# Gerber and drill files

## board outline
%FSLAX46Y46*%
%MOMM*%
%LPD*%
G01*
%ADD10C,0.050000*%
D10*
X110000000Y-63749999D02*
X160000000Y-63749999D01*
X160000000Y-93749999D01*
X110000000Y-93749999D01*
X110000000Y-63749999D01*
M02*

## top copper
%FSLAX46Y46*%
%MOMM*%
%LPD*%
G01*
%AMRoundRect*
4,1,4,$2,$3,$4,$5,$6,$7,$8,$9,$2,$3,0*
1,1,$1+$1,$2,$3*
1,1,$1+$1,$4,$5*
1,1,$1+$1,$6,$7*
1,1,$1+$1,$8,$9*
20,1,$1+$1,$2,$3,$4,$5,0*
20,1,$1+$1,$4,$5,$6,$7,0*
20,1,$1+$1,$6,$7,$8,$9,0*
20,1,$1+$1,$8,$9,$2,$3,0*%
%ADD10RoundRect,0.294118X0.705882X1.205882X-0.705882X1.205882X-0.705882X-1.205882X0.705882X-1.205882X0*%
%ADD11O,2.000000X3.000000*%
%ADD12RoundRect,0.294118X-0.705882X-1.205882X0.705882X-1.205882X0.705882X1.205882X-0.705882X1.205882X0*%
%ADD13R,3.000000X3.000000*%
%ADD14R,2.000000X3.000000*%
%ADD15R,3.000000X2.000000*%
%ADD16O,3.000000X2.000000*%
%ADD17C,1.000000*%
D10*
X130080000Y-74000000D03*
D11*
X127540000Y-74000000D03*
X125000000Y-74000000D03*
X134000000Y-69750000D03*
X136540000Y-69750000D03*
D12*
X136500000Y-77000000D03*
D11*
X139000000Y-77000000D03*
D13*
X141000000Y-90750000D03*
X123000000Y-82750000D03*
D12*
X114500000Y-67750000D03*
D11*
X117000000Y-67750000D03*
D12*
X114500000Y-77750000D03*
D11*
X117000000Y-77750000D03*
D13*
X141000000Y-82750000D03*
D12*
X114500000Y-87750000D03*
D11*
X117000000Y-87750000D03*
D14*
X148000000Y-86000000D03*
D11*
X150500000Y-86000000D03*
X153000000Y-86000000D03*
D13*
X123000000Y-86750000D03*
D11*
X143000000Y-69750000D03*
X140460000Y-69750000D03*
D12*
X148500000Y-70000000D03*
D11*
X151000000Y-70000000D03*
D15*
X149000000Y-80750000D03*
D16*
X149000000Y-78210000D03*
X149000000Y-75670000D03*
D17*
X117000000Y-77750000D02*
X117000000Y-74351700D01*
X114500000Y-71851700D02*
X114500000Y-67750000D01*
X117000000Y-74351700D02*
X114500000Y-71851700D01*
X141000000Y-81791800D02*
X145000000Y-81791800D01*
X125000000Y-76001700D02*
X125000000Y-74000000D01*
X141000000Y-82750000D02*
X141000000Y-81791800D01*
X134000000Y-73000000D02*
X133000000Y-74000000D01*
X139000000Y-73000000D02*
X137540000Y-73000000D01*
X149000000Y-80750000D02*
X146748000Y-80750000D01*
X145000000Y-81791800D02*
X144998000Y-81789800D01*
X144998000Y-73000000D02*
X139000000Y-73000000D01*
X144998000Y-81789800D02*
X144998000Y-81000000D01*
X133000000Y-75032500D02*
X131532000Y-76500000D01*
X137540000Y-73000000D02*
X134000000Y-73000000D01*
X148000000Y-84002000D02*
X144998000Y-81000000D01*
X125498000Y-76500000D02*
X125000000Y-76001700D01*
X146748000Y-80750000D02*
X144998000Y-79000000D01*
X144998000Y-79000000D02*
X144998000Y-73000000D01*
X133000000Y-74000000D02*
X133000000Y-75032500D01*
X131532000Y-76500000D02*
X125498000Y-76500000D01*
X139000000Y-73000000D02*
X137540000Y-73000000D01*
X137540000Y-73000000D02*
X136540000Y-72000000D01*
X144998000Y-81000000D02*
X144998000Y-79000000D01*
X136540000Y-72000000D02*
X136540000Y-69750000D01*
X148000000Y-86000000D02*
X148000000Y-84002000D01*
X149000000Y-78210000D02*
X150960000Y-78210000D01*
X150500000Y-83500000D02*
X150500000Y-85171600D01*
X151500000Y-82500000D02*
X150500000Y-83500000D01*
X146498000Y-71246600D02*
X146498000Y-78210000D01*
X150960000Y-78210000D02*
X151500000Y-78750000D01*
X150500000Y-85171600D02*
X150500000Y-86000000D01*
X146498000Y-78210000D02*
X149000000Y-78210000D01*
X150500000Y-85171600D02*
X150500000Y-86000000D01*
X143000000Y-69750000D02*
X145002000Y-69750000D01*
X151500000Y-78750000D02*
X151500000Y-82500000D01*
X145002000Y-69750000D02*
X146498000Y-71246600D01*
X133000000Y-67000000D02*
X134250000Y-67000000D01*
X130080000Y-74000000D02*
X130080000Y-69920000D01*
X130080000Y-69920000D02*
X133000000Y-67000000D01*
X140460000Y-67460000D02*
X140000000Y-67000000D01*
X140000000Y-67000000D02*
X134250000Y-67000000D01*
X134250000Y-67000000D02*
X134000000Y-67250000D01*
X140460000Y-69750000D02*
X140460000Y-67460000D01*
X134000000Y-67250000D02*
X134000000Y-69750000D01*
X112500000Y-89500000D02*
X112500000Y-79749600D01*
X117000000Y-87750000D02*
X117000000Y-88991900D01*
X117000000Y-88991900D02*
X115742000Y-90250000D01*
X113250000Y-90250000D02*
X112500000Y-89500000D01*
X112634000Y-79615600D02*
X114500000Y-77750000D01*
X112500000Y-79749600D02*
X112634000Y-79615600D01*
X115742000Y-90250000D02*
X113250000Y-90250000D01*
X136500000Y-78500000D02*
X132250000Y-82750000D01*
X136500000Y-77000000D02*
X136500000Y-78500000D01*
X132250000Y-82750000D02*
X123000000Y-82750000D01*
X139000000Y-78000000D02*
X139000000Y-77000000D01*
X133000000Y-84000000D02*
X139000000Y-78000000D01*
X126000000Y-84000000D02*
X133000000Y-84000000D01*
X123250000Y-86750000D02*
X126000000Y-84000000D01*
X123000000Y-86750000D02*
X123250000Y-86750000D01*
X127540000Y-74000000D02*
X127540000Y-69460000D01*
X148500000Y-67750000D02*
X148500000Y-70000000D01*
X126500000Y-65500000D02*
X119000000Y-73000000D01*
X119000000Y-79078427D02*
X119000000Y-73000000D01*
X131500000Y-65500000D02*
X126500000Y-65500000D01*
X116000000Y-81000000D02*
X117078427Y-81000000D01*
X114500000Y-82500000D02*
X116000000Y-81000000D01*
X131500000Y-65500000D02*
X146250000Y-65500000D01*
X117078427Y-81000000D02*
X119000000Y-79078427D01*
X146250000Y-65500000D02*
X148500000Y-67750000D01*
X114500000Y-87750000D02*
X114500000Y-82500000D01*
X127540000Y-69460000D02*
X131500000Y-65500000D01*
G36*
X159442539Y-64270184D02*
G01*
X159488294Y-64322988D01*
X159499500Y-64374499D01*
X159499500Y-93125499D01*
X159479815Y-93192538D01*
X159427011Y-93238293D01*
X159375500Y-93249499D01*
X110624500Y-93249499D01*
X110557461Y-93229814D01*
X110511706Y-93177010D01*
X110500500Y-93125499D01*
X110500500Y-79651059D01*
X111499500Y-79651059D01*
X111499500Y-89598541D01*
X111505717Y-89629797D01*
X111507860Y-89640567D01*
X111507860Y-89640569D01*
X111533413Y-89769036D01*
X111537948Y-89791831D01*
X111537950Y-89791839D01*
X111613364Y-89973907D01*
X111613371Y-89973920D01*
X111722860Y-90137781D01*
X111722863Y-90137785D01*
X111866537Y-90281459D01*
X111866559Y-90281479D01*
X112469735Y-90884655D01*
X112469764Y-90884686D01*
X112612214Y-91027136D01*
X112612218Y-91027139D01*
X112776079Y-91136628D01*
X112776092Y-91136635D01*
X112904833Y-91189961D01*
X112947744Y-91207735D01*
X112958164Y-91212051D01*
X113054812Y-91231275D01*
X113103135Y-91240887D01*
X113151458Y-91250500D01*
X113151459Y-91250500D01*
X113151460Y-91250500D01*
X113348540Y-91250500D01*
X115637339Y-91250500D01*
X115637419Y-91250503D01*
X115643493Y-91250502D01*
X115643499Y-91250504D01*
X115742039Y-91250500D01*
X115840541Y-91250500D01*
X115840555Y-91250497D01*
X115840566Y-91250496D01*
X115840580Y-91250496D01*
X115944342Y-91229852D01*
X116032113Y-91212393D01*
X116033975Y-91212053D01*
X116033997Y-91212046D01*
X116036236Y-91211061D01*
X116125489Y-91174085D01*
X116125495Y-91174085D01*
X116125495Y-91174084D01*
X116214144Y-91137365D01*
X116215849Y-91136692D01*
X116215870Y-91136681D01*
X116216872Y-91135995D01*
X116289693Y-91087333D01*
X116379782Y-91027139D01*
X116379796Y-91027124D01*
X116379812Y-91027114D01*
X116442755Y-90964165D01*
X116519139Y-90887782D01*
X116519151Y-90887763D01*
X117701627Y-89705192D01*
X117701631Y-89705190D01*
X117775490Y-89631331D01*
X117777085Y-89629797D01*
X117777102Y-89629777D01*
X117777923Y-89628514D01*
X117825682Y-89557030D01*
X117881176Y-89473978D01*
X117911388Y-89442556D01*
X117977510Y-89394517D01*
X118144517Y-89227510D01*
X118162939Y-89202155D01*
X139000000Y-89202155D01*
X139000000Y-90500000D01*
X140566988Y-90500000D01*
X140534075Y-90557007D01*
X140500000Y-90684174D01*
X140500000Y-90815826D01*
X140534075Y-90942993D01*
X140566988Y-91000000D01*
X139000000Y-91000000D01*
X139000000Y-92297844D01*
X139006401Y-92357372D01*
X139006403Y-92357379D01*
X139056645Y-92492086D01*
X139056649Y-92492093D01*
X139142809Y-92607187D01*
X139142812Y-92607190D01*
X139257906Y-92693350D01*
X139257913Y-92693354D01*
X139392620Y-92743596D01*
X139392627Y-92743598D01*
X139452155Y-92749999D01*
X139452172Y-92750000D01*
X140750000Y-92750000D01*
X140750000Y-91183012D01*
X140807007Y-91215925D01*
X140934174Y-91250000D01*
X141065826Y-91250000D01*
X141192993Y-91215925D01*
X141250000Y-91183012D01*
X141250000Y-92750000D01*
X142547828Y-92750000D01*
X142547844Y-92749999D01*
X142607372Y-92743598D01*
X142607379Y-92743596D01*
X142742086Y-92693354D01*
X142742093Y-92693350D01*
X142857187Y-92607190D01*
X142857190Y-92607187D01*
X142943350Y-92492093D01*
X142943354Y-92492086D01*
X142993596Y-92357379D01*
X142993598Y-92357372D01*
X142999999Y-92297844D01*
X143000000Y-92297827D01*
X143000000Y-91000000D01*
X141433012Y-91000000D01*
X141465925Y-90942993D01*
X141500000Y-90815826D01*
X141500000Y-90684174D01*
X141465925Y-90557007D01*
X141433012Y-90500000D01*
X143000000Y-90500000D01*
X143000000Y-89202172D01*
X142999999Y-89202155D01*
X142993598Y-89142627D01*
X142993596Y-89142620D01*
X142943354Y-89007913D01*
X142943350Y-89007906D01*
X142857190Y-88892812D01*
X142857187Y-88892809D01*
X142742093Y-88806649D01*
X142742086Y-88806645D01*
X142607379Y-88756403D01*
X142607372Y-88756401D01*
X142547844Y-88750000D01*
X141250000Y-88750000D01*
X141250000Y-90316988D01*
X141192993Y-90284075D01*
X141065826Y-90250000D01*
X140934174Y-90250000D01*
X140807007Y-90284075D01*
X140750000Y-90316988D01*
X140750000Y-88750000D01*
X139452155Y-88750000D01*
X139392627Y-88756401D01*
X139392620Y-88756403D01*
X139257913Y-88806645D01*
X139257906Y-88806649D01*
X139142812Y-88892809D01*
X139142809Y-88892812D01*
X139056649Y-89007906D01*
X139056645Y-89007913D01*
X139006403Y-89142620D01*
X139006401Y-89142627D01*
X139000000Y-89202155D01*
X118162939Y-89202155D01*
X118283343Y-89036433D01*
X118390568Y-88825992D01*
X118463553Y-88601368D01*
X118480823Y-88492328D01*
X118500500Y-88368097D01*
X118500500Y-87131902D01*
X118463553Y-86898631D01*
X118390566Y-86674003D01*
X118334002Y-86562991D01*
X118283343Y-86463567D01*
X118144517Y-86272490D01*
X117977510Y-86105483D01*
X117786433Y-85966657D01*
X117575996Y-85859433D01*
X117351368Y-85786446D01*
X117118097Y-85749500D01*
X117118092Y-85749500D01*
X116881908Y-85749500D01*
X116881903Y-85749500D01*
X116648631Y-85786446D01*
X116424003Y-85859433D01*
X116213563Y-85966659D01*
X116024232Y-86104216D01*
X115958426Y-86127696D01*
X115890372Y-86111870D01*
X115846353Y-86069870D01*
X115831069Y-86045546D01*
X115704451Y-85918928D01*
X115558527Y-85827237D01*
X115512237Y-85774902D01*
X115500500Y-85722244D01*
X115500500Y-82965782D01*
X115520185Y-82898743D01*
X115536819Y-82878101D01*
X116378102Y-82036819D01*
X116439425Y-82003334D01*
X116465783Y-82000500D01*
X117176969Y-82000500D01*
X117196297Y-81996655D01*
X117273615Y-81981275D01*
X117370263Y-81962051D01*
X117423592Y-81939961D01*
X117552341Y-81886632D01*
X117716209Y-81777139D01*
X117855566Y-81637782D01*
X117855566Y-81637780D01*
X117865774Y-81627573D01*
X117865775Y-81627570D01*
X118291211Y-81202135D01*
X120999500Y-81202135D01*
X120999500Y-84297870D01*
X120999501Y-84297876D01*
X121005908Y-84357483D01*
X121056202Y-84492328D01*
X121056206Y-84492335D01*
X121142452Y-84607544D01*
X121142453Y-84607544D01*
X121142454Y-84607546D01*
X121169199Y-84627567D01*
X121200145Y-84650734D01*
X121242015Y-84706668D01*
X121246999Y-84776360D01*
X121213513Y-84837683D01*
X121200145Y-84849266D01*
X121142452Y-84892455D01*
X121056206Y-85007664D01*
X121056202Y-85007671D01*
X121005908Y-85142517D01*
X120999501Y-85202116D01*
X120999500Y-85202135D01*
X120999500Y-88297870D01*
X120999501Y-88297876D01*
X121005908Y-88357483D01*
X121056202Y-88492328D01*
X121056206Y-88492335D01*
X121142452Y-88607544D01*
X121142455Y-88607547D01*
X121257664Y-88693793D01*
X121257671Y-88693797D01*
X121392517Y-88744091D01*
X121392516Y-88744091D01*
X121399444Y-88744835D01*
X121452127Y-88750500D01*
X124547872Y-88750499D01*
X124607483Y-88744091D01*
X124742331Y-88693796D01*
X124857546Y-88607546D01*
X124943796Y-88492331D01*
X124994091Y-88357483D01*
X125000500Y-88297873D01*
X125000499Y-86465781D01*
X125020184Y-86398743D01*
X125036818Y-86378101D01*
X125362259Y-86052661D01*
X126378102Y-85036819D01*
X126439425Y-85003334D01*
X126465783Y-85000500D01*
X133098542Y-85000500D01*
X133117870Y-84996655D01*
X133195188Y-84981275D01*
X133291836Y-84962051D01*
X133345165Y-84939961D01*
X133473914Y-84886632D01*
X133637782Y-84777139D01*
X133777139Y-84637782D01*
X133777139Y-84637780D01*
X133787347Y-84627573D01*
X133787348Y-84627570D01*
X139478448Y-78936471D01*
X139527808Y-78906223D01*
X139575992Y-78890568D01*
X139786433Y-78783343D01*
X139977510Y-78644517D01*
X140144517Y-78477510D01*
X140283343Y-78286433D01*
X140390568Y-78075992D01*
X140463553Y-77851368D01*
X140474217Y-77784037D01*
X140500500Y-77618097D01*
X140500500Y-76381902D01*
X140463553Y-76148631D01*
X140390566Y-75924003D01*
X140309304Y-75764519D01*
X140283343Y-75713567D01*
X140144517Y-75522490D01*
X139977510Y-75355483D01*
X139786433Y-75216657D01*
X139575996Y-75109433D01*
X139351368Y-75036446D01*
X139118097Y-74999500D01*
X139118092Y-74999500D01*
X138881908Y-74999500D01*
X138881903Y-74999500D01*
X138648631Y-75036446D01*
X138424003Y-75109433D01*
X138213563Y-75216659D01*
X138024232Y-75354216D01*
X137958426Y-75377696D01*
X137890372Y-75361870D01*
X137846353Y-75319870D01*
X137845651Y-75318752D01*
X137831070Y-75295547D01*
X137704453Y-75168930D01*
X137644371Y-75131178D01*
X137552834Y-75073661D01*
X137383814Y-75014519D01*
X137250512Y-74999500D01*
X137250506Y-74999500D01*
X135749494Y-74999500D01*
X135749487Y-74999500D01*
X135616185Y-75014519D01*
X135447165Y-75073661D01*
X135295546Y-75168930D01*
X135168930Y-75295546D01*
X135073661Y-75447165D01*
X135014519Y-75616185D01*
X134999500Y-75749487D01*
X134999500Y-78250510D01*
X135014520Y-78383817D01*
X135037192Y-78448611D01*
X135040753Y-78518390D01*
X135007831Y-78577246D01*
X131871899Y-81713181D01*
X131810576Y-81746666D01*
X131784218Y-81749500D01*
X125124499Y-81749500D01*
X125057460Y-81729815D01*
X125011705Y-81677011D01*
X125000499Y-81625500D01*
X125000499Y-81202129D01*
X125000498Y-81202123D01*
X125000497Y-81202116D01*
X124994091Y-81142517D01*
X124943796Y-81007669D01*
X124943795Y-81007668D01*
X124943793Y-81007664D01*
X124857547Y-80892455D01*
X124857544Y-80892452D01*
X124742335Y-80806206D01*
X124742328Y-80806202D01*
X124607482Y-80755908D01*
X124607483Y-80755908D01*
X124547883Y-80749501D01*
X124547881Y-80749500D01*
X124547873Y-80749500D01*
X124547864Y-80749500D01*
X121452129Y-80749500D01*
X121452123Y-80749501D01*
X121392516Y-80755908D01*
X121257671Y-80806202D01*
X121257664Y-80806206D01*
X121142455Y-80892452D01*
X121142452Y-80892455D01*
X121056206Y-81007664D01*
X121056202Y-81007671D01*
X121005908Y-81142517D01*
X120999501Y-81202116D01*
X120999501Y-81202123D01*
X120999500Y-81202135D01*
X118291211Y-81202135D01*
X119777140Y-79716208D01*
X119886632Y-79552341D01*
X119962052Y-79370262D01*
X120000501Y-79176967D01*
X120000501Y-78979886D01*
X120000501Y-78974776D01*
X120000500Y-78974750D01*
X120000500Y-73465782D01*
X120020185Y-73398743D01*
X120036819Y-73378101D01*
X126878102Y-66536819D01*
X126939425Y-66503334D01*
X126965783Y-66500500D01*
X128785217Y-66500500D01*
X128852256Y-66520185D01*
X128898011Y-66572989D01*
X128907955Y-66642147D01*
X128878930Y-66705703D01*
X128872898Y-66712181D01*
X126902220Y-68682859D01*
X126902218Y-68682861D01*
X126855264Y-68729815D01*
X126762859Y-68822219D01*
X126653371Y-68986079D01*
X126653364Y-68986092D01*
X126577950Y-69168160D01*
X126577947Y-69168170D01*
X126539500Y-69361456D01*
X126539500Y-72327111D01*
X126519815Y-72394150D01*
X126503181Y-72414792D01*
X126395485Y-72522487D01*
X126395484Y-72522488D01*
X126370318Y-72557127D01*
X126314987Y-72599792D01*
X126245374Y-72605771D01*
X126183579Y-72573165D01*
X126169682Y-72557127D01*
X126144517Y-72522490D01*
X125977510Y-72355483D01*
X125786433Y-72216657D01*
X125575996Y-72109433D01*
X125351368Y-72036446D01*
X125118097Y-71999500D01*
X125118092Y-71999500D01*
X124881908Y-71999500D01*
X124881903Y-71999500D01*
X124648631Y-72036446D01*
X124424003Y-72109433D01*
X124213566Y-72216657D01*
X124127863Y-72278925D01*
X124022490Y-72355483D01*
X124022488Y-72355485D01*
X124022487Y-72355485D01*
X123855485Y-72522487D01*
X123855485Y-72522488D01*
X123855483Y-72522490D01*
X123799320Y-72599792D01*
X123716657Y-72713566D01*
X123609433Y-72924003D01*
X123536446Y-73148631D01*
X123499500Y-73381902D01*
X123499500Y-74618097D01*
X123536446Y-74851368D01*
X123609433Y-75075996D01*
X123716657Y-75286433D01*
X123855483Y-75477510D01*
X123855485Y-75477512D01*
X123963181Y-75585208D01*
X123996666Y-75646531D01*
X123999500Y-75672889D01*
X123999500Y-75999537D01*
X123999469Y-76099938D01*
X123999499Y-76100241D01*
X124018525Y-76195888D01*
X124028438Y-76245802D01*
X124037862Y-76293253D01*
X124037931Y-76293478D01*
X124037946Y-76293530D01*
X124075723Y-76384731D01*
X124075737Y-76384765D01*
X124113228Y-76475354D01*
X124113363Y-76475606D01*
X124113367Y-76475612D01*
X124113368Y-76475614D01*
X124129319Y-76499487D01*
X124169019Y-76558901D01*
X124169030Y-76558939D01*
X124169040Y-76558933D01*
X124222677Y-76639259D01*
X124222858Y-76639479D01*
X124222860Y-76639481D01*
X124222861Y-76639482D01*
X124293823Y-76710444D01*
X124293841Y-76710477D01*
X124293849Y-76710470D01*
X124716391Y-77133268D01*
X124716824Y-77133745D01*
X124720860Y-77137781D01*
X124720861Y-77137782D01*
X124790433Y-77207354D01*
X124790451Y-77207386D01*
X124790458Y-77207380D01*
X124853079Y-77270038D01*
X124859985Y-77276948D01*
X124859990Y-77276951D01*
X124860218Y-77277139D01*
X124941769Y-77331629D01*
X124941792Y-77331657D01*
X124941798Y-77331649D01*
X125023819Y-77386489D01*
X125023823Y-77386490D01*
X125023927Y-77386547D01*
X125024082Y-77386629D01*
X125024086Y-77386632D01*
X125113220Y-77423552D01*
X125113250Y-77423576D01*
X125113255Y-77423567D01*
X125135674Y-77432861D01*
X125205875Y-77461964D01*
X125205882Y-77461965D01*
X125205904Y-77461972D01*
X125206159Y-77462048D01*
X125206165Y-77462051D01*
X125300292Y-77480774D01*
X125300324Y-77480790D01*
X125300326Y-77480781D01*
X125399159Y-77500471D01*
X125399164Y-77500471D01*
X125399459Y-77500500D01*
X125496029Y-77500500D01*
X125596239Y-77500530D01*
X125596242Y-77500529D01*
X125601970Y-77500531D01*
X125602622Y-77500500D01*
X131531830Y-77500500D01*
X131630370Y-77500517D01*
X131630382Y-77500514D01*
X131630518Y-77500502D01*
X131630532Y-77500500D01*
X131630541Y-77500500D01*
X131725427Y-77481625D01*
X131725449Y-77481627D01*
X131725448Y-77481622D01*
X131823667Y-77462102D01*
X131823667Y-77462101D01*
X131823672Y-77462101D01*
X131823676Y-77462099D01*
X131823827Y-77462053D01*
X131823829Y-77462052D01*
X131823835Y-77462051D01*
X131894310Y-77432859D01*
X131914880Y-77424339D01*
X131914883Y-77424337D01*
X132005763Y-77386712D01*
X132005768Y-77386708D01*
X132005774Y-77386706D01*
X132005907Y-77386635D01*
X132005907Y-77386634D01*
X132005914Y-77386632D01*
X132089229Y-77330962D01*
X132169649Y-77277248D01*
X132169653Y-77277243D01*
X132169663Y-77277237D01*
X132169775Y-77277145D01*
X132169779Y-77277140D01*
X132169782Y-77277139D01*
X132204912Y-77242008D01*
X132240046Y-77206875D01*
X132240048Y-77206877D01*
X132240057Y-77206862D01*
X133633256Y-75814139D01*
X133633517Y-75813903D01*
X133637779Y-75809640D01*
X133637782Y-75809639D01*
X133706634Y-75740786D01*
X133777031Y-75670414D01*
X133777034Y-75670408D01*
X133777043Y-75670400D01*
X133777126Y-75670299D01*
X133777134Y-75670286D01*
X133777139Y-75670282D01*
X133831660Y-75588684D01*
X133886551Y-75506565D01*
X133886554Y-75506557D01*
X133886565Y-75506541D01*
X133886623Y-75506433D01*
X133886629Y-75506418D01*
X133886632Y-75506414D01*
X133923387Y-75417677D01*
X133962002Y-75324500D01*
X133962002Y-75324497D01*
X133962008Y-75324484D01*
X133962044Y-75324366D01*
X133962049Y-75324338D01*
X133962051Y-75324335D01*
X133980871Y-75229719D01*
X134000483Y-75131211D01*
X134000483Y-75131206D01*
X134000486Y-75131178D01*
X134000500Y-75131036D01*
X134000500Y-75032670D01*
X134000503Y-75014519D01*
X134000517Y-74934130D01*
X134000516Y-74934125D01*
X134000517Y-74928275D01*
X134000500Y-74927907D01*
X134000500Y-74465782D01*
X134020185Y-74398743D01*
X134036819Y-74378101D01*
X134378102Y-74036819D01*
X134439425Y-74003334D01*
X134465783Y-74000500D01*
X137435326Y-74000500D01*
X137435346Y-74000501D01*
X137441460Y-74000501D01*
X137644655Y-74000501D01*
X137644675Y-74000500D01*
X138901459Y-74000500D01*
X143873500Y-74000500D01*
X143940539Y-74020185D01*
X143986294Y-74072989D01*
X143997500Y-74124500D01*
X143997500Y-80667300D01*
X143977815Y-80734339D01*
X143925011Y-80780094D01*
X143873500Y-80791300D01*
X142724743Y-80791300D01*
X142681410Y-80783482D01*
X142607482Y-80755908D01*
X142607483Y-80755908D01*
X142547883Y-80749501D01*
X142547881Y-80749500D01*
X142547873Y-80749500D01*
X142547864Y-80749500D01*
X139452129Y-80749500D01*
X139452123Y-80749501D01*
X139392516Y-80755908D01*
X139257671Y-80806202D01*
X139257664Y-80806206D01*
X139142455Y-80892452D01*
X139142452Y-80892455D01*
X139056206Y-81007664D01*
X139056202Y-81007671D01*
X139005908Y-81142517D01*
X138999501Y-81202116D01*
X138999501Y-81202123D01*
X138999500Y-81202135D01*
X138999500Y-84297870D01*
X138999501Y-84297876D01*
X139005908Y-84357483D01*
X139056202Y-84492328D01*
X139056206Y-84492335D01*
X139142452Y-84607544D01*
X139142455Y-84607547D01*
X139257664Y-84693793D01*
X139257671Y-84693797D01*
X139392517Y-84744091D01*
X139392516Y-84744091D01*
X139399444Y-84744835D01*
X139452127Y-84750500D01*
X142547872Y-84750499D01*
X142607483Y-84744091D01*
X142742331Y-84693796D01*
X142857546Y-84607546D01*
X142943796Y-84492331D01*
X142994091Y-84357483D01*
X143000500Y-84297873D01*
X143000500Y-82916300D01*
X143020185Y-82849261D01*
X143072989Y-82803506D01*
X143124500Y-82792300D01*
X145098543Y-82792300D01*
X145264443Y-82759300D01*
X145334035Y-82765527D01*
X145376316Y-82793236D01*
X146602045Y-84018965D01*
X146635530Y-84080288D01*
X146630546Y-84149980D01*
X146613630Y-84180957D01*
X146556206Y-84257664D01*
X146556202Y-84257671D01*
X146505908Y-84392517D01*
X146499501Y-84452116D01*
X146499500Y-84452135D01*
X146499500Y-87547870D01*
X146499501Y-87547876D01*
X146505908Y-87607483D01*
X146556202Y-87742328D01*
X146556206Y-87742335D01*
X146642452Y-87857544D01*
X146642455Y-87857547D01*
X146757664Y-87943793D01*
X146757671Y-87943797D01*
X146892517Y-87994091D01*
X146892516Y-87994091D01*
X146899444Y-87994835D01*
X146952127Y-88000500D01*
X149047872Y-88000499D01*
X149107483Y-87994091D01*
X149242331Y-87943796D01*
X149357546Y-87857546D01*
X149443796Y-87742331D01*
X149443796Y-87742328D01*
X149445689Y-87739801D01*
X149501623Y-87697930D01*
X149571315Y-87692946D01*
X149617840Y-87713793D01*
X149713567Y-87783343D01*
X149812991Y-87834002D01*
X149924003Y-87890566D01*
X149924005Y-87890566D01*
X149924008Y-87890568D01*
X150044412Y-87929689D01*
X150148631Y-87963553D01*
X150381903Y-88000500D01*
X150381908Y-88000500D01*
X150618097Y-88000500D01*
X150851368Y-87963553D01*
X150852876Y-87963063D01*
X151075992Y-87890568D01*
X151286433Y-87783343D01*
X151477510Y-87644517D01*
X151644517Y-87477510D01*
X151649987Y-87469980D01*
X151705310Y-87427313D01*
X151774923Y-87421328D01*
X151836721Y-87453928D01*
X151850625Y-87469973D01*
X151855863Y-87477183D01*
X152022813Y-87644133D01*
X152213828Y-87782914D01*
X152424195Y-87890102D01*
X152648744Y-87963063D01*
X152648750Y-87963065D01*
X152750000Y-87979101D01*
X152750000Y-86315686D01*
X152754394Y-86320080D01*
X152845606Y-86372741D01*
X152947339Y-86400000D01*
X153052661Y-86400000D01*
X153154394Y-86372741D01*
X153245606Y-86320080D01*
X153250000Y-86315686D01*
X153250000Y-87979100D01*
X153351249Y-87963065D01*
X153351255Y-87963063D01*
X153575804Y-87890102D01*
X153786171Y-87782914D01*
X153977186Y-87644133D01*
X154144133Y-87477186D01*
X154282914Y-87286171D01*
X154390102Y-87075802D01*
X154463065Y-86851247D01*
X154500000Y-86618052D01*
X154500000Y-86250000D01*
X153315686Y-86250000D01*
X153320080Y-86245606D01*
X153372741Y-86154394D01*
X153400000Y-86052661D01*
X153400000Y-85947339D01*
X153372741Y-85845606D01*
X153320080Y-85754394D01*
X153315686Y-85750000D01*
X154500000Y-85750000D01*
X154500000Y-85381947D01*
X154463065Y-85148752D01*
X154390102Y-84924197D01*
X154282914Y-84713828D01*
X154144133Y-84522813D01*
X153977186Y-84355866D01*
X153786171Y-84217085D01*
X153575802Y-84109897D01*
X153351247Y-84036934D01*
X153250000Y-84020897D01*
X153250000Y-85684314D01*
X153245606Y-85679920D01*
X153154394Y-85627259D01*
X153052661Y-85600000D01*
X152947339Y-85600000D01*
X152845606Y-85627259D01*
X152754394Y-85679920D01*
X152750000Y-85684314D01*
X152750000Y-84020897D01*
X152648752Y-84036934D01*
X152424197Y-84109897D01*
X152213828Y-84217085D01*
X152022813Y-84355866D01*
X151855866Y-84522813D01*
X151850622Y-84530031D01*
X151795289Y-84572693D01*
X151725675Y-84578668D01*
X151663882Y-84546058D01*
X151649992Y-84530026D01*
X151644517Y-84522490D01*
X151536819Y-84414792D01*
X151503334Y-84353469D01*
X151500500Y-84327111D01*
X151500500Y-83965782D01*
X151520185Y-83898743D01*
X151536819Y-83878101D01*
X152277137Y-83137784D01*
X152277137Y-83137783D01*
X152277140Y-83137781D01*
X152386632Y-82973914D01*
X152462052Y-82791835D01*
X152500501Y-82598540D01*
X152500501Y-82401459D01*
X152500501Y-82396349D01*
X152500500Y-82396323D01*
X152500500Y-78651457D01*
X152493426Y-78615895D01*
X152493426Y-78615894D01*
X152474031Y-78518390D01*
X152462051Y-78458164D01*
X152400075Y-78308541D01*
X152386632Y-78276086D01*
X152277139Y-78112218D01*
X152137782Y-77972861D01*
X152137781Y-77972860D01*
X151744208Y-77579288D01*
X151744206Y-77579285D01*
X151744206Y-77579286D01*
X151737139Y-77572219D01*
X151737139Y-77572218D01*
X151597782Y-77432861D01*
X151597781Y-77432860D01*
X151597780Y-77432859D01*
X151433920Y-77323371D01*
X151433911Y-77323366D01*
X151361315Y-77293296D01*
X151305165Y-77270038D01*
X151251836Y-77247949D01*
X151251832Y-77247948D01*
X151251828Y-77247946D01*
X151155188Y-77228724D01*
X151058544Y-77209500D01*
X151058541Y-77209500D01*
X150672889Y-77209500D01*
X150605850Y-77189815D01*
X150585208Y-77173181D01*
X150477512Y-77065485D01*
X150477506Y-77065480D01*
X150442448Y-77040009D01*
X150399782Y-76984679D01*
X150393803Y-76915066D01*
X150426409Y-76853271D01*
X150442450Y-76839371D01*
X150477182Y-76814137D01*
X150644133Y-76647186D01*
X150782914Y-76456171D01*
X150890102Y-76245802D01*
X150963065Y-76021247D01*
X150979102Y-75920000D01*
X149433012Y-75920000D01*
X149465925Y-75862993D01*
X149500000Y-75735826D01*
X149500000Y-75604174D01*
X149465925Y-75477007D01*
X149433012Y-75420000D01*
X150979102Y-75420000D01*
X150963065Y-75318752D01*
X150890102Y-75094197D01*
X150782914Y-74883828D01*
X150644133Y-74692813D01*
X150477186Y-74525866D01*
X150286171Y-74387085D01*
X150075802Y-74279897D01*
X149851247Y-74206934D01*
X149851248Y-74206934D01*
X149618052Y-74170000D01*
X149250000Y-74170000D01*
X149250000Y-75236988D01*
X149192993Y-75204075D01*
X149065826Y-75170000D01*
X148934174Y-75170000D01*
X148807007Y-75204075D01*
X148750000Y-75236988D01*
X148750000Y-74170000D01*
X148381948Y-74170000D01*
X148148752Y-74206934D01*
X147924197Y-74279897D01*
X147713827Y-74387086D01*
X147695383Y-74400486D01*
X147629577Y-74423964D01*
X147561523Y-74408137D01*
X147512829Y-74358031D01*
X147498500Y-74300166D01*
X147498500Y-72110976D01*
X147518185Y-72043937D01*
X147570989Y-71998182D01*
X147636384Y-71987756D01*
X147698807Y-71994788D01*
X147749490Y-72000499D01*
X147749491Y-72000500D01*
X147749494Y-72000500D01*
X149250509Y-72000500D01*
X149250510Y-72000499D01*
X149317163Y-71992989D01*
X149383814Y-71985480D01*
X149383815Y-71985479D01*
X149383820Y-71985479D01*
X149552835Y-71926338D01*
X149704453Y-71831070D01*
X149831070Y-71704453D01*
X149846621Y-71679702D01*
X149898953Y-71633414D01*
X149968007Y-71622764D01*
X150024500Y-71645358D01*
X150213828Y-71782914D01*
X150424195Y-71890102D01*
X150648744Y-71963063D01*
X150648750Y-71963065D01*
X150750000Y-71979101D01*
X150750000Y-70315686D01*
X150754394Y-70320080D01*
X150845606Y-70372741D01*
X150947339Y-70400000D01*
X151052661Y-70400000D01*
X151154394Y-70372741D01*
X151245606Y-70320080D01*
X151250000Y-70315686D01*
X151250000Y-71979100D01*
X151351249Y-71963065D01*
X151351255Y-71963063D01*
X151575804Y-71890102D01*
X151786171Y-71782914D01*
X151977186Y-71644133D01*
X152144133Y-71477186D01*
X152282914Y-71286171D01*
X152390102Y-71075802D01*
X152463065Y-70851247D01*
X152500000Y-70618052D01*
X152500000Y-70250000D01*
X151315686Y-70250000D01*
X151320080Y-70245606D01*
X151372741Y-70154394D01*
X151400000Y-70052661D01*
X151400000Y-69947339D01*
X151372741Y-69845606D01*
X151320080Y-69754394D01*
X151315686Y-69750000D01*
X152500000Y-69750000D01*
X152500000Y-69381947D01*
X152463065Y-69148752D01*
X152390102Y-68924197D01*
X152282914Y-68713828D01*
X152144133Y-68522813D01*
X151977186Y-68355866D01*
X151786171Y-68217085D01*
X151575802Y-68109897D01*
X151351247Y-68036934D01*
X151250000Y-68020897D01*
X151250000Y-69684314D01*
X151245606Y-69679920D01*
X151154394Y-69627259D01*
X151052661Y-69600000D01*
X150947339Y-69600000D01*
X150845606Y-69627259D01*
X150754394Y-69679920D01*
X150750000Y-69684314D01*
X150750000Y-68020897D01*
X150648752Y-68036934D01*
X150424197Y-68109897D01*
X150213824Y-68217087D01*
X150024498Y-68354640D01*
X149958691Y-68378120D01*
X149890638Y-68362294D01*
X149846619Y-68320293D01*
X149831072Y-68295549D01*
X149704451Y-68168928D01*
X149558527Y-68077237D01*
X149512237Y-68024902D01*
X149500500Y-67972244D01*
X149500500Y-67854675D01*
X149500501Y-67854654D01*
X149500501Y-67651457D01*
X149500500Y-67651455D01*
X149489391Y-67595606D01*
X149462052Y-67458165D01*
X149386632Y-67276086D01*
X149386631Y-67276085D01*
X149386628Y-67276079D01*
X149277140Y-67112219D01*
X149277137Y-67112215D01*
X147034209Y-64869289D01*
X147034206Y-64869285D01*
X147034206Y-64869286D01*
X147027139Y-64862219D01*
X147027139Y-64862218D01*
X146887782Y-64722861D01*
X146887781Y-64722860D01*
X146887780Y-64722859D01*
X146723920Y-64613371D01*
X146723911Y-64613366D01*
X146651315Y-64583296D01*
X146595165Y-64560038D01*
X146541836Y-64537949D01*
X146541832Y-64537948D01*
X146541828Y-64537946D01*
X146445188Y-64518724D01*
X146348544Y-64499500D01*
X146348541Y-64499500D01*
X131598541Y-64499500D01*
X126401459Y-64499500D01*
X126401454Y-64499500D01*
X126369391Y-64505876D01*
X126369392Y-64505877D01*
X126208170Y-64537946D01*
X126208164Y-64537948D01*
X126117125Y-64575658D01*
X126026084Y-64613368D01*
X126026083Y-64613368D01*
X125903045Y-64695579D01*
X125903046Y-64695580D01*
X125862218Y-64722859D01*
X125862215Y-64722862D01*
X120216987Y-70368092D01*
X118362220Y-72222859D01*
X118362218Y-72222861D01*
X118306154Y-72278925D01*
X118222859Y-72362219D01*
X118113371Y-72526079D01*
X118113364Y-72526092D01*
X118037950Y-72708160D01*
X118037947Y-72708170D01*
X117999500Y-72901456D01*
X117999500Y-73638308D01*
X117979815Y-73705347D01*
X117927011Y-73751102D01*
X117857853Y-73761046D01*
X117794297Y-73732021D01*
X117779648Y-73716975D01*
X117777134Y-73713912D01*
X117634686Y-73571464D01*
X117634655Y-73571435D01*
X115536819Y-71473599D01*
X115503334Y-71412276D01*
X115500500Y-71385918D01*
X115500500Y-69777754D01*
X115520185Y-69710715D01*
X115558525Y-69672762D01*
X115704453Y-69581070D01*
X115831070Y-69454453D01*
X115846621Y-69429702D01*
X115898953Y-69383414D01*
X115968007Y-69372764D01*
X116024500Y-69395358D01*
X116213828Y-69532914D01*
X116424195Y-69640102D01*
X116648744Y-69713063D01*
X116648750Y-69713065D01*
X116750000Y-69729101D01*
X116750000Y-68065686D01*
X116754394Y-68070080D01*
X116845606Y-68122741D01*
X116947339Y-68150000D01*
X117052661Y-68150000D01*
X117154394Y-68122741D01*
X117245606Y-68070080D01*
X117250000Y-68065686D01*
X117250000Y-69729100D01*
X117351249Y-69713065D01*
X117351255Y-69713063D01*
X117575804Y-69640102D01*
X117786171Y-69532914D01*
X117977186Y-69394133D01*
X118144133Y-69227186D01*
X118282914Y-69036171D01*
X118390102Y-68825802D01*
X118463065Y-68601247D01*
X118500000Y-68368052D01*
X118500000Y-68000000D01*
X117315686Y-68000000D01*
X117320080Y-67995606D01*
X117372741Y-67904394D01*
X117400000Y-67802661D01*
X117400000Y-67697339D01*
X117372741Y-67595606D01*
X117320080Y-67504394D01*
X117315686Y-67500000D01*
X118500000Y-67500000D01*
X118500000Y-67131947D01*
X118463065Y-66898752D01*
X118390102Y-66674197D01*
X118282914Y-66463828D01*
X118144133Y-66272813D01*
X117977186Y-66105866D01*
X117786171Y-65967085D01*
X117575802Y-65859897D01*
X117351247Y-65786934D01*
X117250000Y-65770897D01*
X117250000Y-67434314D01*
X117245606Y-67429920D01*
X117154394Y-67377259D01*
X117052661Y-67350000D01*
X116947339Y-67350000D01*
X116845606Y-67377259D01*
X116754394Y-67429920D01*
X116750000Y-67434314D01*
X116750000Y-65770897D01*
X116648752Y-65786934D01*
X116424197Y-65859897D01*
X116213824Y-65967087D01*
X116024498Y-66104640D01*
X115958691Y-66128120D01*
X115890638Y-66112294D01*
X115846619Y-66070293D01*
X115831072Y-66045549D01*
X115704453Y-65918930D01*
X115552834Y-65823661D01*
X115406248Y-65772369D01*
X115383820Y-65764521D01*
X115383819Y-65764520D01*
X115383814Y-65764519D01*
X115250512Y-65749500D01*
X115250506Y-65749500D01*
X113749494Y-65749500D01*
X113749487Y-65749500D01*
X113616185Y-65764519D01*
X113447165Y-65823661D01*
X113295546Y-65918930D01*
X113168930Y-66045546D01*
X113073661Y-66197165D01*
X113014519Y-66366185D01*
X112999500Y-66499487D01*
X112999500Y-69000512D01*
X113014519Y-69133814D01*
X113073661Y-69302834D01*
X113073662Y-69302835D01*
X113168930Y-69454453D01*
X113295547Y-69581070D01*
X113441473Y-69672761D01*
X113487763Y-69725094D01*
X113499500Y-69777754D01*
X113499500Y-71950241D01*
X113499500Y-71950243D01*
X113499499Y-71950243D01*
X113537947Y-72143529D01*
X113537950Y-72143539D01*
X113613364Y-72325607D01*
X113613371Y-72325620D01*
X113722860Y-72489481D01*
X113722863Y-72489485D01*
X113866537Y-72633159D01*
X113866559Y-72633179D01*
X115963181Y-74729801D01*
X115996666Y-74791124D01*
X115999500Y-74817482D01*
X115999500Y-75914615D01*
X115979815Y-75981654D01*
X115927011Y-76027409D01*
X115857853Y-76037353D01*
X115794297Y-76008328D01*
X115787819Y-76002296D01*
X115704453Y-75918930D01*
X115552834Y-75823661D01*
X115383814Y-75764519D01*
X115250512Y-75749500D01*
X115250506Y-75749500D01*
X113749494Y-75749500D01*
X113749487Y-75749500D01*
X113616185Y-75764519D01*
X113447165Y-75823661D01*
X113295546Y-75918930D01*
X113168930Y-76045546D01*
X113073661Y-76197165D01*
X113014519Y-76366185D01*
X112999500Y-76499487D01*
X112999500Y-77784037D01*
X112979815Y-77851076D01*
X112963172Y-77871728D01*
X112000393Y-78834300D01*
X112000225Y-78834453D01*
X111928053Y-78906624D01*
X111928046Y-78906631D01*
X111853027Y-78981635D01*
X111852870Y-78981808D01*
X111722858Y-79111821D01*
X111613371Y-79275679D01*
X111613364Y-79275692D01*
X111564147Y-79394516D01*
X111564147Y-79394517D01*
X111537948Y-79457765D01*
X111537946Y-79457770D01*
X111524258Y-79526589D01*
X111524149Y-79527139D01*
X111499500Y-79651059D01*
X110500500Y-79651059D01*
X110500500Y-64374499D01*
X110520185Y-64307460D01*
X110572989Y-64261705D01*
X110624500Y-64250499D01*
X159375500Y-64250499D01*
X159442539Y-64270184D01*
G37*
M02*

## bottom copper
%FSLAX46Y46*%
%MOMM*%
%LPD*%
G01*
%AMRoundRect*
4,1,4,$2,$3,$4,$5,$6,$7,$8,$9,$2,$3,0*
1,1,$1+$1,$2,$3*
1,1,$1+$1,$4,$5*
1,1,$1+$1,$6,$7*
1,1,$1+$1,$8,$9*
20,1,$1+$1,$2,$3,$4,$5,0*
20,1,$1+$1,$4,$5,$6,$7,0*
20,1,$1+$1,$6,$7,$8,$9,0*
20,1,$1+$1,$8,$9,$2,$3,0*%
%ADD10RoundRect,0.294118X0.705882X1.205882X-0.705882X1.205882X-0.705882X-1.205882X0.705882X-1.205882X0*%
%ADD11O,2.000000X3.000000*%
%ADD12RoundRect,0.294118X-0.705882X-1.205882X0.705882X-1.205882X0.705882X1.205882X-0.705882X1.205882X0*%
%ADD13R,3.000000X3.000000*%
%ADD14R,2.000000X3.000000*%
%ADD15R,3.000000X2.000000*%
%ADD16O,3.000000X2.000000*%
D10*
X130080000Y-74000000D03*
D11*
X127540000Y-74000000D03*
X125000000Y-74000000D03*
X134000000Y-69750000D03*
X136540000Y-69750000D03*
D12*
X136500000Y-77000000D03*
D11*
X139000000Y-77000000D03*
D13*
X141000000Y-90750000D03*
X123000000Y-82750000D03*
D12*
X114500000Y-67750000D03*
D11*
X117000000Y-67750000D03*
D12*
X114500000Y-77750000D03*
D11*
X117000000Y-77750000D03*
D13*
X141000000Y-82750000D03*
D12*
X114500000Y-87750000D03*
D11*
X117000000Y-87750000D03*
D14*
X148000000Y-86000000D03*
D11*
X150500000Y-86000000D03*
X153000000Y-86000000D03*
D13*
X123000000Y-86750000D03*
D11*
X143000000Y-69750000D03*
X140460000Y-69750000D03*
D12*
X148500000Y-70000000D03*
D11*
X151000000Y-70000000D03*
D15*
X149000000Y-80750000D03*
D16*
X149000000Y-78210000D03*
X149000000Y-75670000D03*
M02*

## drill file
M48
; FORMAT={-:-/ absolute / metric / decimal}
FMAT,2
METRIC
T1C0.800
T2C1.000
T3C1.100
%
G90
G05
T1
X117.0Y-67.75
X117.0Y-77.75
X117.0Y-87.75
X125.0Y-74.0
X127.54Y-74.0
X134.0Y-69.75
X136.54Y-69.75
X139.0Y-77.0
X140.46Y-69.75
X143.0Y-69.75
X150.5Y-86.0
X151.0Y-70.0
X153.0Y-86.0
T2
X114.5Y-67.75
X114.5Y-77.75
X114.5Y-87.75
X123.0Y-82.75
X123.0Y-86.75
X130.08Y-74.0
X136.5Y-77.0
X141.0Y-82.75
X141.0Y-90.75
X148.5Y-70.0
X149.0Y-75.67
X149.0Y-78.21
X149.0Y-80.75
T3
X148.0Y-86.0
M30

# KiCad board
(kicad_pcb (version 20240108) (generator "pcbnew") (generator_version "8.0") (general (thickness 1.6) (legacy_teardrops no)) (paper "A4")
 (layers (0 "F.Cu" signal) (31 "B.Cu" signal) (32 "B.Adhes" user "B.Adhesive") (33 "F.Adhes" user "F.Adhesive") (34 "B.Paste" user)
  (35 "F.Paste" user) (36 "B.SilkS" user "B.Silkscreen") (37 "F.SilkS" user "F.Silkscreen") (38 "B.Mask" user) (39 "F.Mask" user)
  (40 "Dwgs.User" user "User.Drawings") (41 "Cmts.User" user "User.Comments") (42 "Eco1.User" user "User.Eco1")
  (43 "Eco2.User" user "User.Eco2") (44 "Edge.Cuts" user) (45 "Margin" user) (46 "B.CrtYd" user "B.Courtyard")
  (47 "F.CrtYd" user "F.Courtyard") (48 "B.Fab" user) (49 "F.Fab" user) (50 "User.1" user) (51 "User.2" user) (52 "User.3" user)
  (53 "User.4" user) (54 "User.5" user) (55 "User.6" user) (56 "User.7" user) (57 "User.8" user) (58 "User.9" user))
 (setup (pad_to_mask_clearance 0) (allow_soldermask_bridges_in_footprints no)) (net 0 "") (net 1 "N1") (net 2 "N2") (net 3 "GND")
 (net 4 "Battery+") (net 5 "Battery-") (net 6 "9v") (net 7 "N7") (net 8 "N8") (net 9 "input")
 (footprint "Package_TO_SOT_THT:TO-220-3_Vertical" (layer "F.Cu") (at 130.08 74 180)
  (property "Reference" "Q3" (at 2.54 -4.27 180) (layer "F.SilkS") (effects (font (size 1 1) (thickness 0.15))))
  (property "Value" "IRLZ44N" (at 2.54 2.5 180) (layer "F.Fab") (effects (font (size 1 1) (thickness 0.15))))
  (pad "1" thru_hole roundrect (at 0 0 180) (size 2 3) (drill 1) (layers "*.Cu" "*.Mask") (remove_unused_layers no)
   (roundrect_rratio 0.147059) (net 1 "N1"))
  (pad "2" thru_hole oval (at 2.54 0 180) (size 2 3) (drill 0.8) (layers "*.Cu" "*.Mask") (remove_unused_layers no) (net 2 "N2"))
  (pad "3" thru_hole oval (at 5.08 0 180) (size 2 3) (drill 0.8) (layers "*.Cu" "*.Mask") (remove_unused_layers no) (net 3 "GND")))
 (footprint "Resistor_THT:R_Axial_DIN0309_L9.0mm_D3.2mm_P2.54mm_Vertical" (layer "F.Cu") (at 134 69.75)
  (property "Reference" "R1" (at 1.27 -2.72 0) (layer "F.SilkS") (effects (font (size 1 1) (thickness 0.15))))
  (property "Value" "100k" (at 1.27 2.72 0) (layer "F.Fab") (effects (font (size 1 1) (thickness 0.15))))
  (pad "1" thru_hole oval (at 0 0) (size 2 3) (drill 0.8) (layers "*.Cu" "*.Mask") (remove_unused_layers no) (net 1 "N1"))
  (pad "2" thru_hole oval (at 2.54 0) (size 2 3) (drill 0.8) (layers "*.Cu" "*.Mask") (remove_unused_layers no) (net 3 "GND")))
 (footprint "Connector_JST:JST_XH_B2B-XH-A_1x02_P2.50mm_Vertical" (layer "F.Cu") (at 136.5 77)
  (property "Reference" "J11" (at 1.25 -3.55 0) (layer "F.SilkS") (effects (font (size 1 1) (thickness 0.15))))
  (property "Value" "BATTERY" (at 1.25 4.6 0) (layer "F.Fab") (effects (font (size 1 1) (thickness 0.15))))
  (pad "1" thru_hole roundrect (at 0 0) (size 2 3) (drill 1) (layers "*.Cu" "*.Mask") (remove_unused_layers no) (roundrect_rratio 0.147059)
   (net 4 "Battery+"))
  (pad "2" thru_hole oval (at 2.5 0) (size 2 3) (drill 0.8) (layers "*.Cu" "*.Mask") (remove_unused_layers no) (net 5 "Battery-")))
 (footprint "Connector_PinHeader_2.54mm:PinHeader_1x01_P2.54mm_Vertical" (layer "F.Cu") (at 141 90.75)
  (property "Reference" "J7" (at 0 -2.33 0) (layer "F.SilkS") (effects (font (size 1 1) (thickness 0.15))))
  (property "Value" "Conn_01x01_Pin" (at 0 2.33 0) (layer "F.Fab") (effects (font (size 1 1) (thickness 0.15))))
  (pad "1" thru_hole rect (at 0 0) (size 3 3) (drill 1) (layers "*.Cu" "*.Mask") (remove_unused_layers no) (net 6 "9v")))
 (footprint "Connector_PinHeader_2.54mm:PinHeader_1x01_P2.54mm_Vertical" (layer "F.Cu") (at 123 82.75 90)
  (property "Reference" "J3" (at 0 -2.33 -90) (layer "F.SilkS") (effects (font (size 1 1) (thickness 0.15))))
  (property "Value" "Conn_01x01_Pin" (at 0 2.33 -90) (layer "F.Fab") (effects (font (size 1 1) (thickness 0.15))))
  (pad "1" thru_hole rect (at 0 0 90) (size 3 3) (drill 1) (layers "*.Cu" "*.Mask") (remove_unused_layers no) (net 4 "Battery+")))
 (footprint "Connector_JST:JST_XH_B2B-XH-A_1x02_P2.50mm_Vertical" (layer "F.Cu") (at 114.5 67.75)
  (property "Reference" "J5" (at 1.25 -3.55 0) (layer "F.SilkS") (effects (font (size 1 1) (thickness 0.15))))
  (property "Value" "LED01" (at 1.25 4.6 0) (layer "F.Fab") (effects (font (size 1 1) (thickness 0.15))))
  (pad "1" thru_hole roundrect (at 0 0) (size 2 3) (drill 1) (layers "*.Cu" "*.Mask") (remove_unused_layers no) (roundrect_rratio 0.147059)
   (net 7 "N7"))
  (pad "2" thru_hole oval (at 2.5 0) (size 2 3) (drill 0.8) (layers "*.Cu" "*.Mask") (remove_unused_layers no) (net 6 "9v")))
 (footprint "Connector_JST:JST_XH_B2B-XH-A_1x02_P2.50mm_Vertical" (layer "F.Cu") (at 114.5 77.75)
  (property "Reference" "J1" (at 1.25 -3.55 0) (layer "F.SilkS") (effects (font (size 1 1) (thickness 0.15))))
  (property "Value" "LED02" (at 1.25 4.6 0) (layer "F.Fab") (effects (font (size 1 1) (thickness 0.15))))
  (pad "1" thru_hole roundrect (at 0 0) (size 2 3) (drill 1) (layers "*.Cu" "*.Mask") (remove_unused_layers no) (roundrect_rratio 0.147059)
   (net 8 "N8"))
  (pad "2" thru_hole oval (at 2.5 0) (size 2 3) (drill 0.8) (layers "*.Cu" "*.Mask") (remove_unused_layers no) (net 7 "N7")))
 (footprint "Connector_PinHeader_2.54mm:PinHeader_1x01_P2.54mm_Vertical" (layer "F.Cu") (at 141 82.75)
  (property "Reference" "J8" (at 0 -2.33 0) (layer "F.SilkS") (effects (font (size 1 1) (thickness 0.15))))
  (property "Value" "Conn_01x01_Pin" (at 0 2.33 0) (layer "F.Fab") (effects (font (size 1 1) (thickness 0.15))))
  (pad "1" thru_hole rect (at 0 0) (size 3 3) (drill 1) (layers "*.Cu" "*.Mask") (remove_unused_layers no) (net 3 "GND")))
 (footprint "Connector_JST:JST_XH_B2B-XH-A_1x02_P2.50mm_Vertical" (layer "F.Cu") (at 114.5 87.75)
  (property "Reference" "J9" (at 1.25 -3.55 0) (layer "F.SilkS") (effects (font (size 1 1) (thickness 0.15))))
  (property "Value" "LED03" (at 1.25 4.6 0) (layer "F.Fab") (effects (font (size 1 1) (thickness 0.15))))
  (pad "1" thru_hole roundrect (at 0 0) (size 2 3) (drill 1) (layers "*.Cu" "*.Mask") (remove_unused_layers no) (roundrect_rratio 0.147059)
   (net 2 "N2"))
  (pad "2" thru_hole oval (at 2.5 0) (size 2 3) (drill 0.8) (layers "*.Cu" "*.Mask") (remove_unused_layers no) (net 8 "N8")))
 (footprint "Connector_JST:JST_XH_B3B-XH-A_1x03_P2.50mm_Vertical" (layer "F.Cu") (at 148 86)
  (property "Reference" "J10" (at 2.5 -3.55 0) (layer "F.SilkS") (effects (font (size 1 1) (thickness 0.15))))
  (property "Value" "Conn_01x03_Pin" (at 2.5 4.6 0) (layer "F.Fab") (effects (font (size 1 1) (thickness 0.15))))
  (pad "1" thru_hole rect (at 0 0) (size 2 3) (drill 1.1) (layers "*.Cu" "*.Mask") (remove_unused_layers no) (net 3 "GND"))
  (pad "2" thru_hole oval (at 2.5 0) (size 2 3) (drill 0.8) (layers "*.Cu" "*.Mask") (remove_unused_layers no) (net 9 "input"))
  (pad "3" thru_hole oval (at 5 0) (size 2 3) (drill 0.8) (layers "*.Cu" "*.Mask") (remove_unused_layers no) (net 6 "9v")))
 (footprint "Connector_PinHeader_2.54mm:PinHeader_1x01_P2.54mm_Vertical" (layer "F.Cu") (at 123 86.75 90)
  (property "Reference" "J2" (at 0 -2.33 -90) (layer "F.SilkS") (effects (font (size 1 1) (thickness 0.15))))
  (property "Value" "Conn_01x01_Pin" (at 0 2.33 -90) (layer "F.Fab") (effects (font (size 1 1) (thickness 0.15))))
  (pad "1" thru_hole rect (at 0 0 90) (size 3 3) (drill 1) (layers "*.Cu" "*.Mask") (remove_unused_layers no) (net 5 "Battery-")))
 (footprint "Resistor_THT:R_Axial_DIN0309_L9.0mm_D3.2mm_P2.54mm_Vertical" (layer "F.Cu") (at 143 69.75 180)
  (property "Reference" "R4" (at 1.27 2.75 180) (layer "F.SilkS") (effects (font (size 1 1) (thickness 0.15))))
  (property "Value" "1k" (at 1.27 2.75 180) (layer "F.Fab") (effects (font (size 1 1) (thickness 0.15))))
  (pad "1" thru_hole oval (at 0 0 180) (size 2 3) (drill 0.8) (layers "*.Cu" "*.Mask") (remove_unused_layers no) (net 9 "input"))
  (pad "2" thru_hole oval (at 2.54 0 180) (size 2 3) (drill 0.8) (layers "*.Cu" "*.Mask") (remove_unused_layers no) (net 1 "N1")))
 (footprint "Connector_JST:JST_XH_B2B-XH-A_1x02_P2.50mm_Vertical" (layer "F.Cu") (at 148.5 70)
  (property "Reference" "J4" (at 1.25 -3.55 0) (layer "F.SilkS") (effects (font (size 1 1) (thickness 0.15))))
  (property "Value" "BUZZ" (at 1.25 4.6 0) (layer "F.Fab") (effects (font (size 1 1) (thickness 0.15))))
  (pad "1" thru_hole roundrect (at 0 0) (size 2 3) (drill 1) (layers "*.Cu" "*.Mask") (remove_unused_layers no) (roundrect_rratio 0.147059)
   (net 2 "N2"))
  (pad "2" thru_hole oval (at 2.5 0) (size 2 3) (drill 0.8) (layers "*.Cu" "*.Mask") (remove_unused_layers no) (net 6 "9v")))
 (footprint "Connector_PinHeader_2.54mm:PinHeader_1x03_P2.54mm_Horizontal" (layer "B.Cu") (at 149 80.75)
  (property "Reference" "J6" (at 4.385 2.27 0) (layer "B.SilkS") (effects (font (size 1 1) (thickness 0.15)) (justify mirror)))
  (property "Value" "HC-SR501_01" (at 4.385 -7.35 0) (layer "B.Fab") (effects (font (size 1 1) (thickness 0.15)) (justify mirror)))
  (pad "1" thru_hole rect (at 0 0) (size 3 2) (drill 1) (layers "*.Cu" "*.Mask") (remove_unused_layers no) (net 3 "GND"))
  (pad "2" thru_hole oval (at 0 -2.54) (size 3 2) (drill 1) (layers "*.Cu" "*.Mask") (remove_unused_layers no) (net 9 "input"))
  (pad "3" thru_hole oval (at 0 -5.08) (size 3 2) (drill 1) (layers "*.Cu" "*.Mask") (remove_unused_layers no) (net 6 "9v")))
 (gr_rect (start 110 63.749999) (end 160 93.749999) (stroke (width 0.05) (type default)) (fill none) (layer "Edge.Cuts"))
 (segment (start 117 77.75) (end 117 74.3517) (width 1) (layer "F.Cu") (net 7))
 (segment (start 114.5 71.8517) (end 114.5 67.75) (width 1) (layer "F.Cu") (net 7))
 (segment (start 117 74.3517) (end 114.5 71.8517) (width 1) (layer "F.Cu") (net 7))
 (segment (start 141 81.7918) (end 145 81.7918) (width 1) (layer "F.Cu") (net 3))
 (segment (start 125 76.0017) (end 125 74) (width 1) (layer "F.Cu") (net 3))
 (segment (start 141 82.75) (end 141 81.7918) (width 1) (layer "F.Cu") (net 3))
 (segment (start 134 73) (end 133 74) (width 1) (layer "F.Cu") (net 3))
 (segment (start 139 73) (end 137.54 73) (width 1) (layer "F.Cu") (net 3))
 (segment (start 149 80.75) (end 146.748 80.75) (width 1) (layer "F.Cu") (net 3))
 (segment (start 145 81.7918) (end 144.998 81.7898) (width 1) (layer "F.Cu") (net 3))
 (segment (start 144.998 73) (end 139 73) (width 1) (layer "F.Cu") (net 3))
 (segment (start 144.998 81.7898) (end 144.998 81) (width 1) (layer "F.Cu") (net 3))
 (segment (start 133 75.0325) (end 131.532 76.5) (width 1) (layer "F.Cu") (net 3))
 (segment (start 137.54 73) (end 134 73) (width 1) (layer "F.Cu") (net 3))
 (segment (start 148 84.002) (end 144.998 81) (width 1) (layer "F.Cu") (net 3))
 (segment (start 125.498 76.5) (end 125 76.0017) (width 1) (layer "F.Cu") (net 3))
 (segment (start 146.748 80.75) (end 144.998 79) (width 1) (layer "F.Cu") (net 3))
 (segment (start 144.998 79) (end 144.998 73) (width 1) (layer "F.Cu") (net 3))
 (segment (start 133 74) (end 133 75.0325) (width 1) (layer "F.Cu") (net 3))
 (segment (start 131.532 76.5) (end 125.498 76.5) (width 1) (layer "F.Cu") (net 3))
 (segment (start 139 73) (end 137.54 73) (width 1) (layer "F.Cu") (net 3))
 (segment (start 137.54 73) (end 136.54 72) (width 1) (layer "F.Cu") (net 3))
 (segment (start 144.998 81) (end 144.998 79) (width 1) (layer "F.Cu") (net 3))
 (segment (start 136.54 72) (end 136.54 69.75) (width 1) (layer "F.Cu") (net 3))
 (segment (start 148 86) (end 148 84.002) (width 1) (layer "F.Cu") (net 3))
 (segment (start 149 78.21) (end 150.96 78.21) (width 1) (layer "F.Cu") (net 9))
 (segment (start 150.5 83.5) (end 150.5 85.1716) (width 1) (layer "F.Cu") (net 9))
 (segment (start 151.5 82.5) (end 150.5 83.5) (width 1) (layer "F.Cu") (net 9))
 (segment (start 146.498 71.2466) (end 146.498 78.21) (width 1) (layer "F.Cu") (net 9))
 (segment (start 150.96 78.21) (end 151.5 78.75) (width 1) (layer "F.Cu") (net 9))
 (segment (start 150.5 85.1716) (end 150.5 86) (width 1) (layer "F.Cu") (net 9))
 (segment (start 146.498 78.21) (end 149 78.21) (width 1) (layer "F.Cu") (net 9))
 (segment (start 150.5 85.1716) (end 150.5 86) (width 1) (layer "F.Cu") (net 9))
 (segment (start 143 69.75) (end 145.002 69.75) (width 1) (layer "F.Cu") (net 9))
 (segment (start 151.5 78.75) (end 151.5 82.5) (width 1) (layer "F.Cu") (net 9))
 (segment (start 145.002 69.75) (end 146.498 71.2466) (width 1) (layer "F.Cu") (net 9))
 (segment (start 133 67) (end 134.25 67) (width 1) (layer "F.Cu") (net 1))
 (segment (start 130.08 74) (end 130.08 69.92) (width 1) (layer "F.Cu") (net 1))
 (segment (start 130.08 69.92) (end 133 67) (width 1) (layer "F.Cu") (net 1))
 (segment (start 140.46 67.46) (end 140 67) (width 1) (layer "F.Cu") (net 1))
 (segment (start 140 67) (end 134.25 67) (width 1) (layer "F.Cu") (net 1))
 (segment (start 134.25 67) (end 134 67.25) (width 1) (layer "F.Cu") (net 1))
 (segment (start 140.46 69.75) (end 140.46 67.46) (width 1) (layer "F.Cu") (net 1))
 (segment (start 134 67.25) (end 134 69.75) (width 1) (layer "F.Cu") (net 1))
 (segment (start 112.5 89.5) (end 112.5 79.7496) (width 1) (layer "F.Cu") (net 8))
 (segment (start 117 87.75) (end 117 88.9919) (width 1) (layer "F.Cu") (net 8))
 (segment (start 117 88.9919) (end 115.742 90.25) (width 1) (layer "F.Cu") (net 8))
 (segment (start 113.25 90.25) (end 112.5 89.5) (width 1) (layer "F.Cu") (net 8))
 (segment (start 112.634 79.6156) (end 114.5 77.75) (width 1) (layer "F.Cu") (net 8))
 (segment (start 112.5 79.7496) (end 112.634 79.6156) (width 1) (layer "F.Cu") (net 8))
 (segment (start 115.742 90.25) (end 113.25 90.25) (width 1) (layer "F.Cu") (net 8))
 (segment (start 136.5 78.5) (end 132.25 82.75) (width 1) (layer "F.Cu") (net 4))
 (segment (start 136.5 77) (end 136.5 78.5) (width 1) (layer "F.Cu") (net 4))
 (segment (start 132.25 82.75) (end 123 82.75) (width 1) (layer "F.Cu") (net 4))
 (segment (start 139 78) (end 139 77) (width 1) (layer "F.Cu") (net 5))
 (segment (start 133 84) (end 139 78) (width 1) (layer "F.Cu") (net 5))
 (segment (start 126 84) (end 133 84) (width 1) (layer "F.Cu") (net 5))
 (segment (start 123.25 86.75) (end 126 84) (width 1) (layer "F.Cu") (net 5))
 (segment (start 123 86.75) (end 123.25 86.75) (width 1) (layer "F.Cu") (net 5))
 (segment (start 127.54 74) (end 127.54 69.46) (width 1) (layer "F.Cu") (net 2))
 (segment (start 148.5 67.75) (end 148.5 70) (width 1) (layer "F.Cu") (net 2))
 (segment (start 126.5 65.5) (end 119 73) (width 1) (layer "F.Cu") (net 2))
 (segment (start 119 79.078427) (end 119 73) (width 1) (layer "F.Cu") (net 2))
 (segment (start 131.5 65.5) (end 126.5 65.5) (width 1) (layer "F.Cu") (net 2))
 (segment (start 116 81) (end 117.078427 81) (width 1) (layer "F.Cu") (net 2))
 (segment (start 114.5 82.5) (end 116 81) (width 1) (layer "F.Cu") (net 2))
 (segment (start 131.5 65.5) (end 146.25 65.5) (width 1) (layer "F.Cu") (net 2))
 (segment (start 117.078427 81) (end 119 79.078427) (width 1) (layer "F.Cu") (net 2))
 (segment (start 146.25 65.5) (end 148.5 67.75) (width 1) (layer "F.Cu") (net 2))
 (segment (start 114.5 87.75) (end 114.5 82.5) (width 1) (layer "F.Cu") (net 2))
 (segment (start 127.54 69.46) (end 131.5 65.5) (width 1) (layer "F.Cu") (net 2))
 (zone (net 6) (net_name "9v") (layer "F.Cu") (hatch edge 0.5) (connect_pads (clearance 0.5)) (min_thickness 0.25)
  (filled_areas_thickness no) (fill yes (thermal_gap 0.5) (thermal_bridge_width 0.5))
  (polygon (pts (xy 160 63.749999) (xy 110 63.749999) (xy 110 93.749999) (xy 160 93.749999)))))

